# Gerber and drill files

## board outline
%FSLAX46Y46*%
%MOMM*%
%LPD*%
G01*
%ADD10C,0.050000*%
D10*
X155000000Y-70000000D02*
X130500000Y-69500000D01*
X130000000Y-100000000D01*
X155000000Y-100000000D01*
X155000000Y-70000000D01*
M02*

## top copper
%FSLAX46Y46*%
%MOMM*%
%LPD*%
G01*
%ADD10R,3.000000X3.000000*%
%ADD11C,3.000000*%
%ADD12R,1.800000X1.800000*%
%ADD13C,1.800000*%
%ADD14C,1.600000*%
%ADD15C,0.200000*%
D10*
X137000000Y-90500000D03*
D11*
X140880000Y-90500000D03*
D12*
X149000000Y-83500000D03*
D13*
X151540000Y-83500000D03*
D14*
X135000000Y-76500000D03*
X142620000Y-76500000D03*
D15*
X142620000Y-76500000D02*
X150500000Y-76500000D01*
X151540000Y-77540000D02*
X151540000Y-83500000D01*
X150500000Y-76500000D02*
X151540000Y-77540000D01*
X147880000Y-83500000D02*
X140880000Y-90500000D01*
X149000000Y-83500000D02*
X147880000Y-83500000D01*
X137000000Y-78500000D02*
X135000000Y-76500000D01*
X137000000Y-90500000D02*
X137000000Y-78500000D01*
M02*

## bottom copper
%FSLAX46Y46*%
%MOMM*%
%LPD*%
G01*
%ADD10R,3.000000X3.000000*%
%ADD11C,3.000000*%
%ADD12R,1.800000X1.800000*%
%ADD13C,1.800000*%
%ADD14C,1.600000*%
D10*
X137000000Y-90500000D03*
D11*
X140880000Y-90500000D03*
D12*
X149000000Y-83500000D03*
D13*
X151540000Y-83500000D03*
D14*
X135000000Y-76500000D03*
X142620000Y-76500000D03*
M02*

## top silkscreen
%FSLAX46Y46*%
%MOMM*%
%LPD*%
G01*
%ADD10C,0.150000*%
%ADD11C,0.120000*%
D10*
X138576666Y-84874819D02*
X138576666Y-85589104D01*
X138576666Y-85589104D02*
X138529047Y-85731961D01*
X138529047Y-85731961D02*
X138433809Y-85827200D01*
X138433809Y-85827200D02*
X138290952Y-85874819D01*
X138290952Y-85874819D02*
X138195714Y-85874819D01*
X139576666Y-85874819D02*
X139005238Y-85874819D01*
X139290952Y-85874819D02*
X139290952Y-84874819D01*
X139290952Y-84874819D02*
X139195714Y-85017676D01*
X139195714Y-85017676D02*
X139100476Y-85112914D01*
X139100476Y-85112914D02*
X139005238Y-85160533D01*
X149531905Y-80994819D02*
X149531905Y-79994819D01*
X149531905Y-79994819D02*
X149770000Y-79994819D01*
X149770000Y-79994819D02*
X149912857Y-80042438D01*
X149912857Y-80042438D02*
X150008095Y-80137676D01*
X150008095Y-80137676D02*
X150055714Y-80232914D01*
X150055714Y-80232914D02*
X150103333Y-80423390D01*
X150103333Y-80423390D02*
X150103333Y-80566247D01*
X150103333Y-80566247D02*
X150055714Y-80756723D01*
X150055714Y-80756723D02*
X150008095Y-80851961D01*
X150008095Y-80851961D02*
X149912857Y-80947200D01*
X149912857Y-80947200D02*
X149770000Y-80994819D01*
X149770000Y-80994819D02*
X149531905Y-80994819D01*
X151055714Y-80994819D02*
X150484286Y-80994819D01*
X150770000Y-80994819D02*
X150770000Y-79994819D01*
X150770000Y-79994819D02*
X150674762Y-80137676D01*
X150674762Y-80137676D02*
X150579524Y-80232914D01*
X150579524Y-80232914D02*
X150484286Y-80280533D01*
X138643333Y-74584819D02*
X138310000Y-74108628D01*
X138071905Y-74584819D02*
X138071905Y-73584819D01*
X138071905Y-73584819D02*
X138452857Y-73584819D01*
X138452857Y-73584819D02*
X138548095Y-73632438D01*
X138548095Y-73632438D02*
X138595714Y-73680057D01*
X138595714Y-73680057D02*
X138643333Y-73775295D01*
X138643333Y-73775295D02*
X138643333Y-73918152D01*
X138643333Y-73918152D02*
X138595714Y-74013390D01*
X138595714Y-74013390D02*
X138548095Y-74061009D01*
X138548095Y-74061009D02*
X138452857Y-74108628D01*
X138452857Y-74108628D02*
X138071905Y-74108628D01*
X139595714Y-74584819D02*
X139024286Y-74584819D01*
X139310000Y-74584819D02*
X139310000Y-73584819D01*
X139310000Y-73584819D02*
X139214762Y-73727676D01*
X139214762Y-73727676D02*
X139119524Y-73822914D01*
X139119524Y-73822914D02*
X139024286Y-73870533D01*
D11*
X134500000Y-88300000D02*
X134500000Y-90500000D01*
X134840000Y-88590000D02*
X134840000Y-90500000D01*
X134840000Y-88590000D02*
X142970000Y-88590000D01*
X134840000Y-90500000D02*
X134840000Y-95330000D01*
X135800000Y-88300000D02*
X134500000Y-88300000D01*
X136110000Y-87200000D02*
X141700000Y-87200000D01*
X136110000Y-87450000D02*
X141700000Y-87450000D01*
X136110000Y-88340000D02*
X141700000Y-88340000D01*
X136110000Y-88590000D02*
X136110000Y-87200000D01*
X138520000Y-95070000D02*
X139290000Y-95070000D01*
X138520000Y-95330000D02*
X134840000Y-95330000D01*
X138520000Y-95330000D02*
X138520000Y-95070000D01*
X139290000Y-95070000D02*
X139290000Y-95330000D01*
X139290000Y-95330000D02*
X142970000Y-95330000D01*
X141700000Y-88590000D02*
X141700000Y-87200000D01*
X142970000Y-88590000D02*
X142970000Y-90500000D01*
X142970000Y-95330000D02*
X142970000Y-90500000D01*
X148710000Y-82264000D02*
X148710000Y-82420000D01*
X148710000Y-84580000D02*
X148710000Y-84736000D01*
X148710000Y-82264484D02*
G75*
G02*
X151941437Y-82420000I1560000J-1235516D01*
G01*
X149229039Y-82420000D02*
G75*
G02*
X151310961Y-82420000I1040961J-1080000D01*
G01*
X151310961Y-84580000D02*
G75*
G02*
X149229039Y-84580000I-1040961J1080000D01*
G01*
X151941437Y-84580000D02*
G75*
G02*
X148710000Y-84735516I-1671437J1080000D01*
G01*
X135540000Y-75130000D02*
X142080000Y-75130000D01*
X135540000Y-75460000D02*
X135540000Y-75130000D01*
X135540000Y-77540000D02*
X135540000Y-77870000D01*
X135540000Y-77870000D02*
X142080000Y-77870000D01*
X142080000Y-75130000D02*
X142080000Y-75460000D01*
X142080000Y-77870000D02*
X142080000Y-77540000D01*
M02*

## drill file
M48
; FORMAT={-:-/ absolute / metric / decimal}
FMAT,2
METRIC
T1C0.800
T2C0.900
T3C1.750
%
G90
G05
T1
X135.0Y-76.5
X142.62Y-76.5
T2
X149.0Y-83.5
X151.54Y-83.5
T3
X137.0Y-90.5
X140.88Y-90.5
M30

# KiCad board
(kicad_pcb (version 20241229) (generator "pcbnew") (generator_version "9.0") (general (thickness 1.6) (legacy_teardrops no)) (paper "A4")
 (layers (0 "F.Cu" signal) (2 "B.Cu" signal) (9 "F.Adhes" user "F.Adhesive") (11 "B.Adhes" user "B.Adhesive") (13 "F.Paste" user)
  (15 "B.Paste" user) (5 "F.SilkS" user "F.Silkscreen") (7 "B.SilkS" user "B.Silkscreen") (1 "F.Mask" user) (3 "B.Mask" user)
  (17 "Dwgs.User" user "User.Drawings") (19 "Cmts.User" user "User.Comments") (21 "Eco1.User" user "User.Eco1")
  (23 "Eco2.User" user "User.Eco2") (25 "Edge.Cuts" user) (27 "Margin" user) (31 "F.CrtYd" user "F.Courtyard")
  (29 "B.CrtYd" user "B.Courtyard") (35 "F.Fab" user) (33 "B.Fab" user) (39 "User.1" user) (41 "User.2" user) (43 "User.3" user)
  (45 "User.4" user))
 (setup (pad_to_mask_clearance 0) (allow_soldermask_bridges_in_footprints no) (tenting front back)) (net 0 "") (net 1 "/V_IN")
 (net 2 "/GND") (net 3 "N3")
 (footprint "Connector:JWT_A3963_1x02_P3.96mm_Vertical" (layer "F.Cu") (at 137 90.5)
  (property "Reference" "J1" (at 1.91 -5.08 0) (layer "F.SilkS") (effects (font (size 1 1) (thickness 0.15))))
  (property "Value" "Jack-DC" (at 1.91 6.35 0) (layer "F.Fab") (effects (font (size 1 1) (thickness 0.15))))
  (fp_line (start -2.5 -2.2) (end -2.5 0) (stroke (width 0.12) (type solid)) (layer "F.SilkS"))
  (fp_line (start -2.16 -1.91) (end -2.16 0) (stroke (width 0.12) (type solid)) (layer "F.SilkS"))
  (fp_line (start -2.16 -1.91) (end 5.97 -1.91) (stroke (width 0.12) (type solid)) (layer "F.SilkS"))
  (fp_line (start -2.16 0) (end -2.16 4.83) (stroke (width 0.12) (type solid)) (layer "F.SilkS"))
  (fp_line (start -1.2 -2.2) (end -2.5 -2.2) (stroke (width 0.12) (type solid)) (layer "F.SilkS"))
  (fp_line (start -0.89 -3.3) (end 4.7 -3.3) (stroke (width 0.12) (type solid)) (layer "F.SilkS"))
  (fp_line (start -0.89 -3.05) (end 4.7 -3.05) (stroke (width 0.12) (type solid)) (layer "F.SilkS"))
  (fp_line (start -0.89 -2.16) (end 4.7 -2.16) (stroke (width 0.12) (type solid)) (layer "F.SilkS"))
  (fp_line (start -0.89 -1.91) (end -0.89 -3.3) (stroke (width 0.12) (type solid)) (layer "F.SilkS"))
  (fp_line (start 1.52 4.57) (end 2.29 4.57) (stroke (width 0.12) (type solid)) (layer "F.SilkS"))
  (fp_line (start 1.52 4.83) (end -2.16 4.83) (stroke (width 0.12) (type solid)) (layer "F.SilkS"))
  (fp_line (start 1.52 4.83) (end 1.52 4.57) (stroke (width 0.12) (type solid)) (layer "F.SilkS"))
  (fp_line (start 2.29 4.57) (end 2.29 4.83) (stroke (width 0.12) (type solid)) (layer "F.SilkS"))
  (fp_line (start 2.29 4.83) (end 5.97 4.83) (stroke (width 0.12) (type solid)) (layer "F.SilkS"))
  (fp_line (start 4.7 -1.91) (end 4.7 -3.3) (stroke (width 0.12) (type solid)) (layer "F.SilkS"))
  (fp_line (start 5.97 -1.91) (end 5.97 0) (stroke (width 0.12) (type solid)) (layer "F.SilkS"))
  (fp_line (start 5.97 4.83) (end 5.97 0) (stroke (width 0.12) (type solid)) (layer "F.SilkS"))
  (pad "1" thru_hole rect (at 0 0) (size 3 3) (drill 1.75) (layers "*.Cu" "*.Mask") (remove_unused_layers no) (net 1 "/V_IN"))
  (pad "2" thru_hole circle (at 3.88 0) (size 3 3) (drill 1.75) (layers "*.Cu" "*.Mask") (remove_unused_layers no) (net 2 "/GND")))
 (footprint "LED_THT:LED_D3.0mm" (layer "F.Cu") (at 149 83.5)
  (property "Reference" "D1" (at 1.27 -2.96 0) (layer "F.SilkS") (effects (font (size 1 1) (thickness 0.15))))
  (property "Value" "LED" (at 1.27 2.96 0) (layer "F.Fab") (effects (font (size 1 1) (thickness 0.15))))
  (fp_line (start -0.29 -1.236) (end -0.29 -1.08) (stroke (width 0.12) (type solid)) (layer "F.SilkS"))
  (fp_line (start -0.29 1.08) (end -0.29 1.236) (stroke (width 0.12) (type solid)) (layer "F.SilkS"))
  (fp_arc (start -0.29 -1.235516) (mid 1.36566 -1.987699) (end 2.941437 -1.08) (stroke (width 0.12) (type solid)) (layer "F.SilkS"))
  (fp_arc (start 0.229039 -1.08) (mid 1.27 -1.5) (end 2.310961 -1.08) (stroke (width 0.12) (type solid)) (layer "F.SilkS"))
  (fp_arc (start 2.310961 1.08) (mid 1.27 1.5) (end 0.229039 1.08) (stroke (width 0.12) (type solid)) (layer "F.SilkS"))
  (fp_arc (start 2.941437 1.08) (mid 1.36566 1.987699) (end -0.29 1.235516) (stroke (width 0.12) (type solid)) (layer "F.SilkS"))
  (pad "1" thru_hole rect (at 0 0) (size 1.8 1.8) (drill 0.9) (layers "*.Cu" "*.Mask") (remove_unused_layers no) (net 2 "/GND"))
  (pad "2" thru_hole circle (at 2.54 0) (size 1.8 1.8) (drill 0.9) (layers "*.Cu" "*.Mask") (remove_unused_layers no) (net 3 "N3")))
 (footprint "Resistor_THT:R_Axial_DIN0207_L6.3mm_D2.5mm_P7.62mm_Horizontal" (layer "F.Cu") (at 135 76.5)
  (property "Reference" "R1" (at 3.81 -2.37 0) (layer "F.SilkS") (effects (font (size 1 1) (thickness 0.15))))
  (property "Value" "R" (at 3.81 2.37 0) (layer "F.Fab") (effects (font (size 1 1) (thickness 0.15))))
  (fp_line (start 0.54 -1.37) (end 7.08 -1.37) (stroke (width 0.12) (type solid)) (layer "F.SilkS"))
  (fp_line (start 0.54 -1.04) (end 0.54 -1.37) (stroke (width 0.12) (type solid)) (layer "F.SilkS"))
  (fp_line (start 0.54 1.04) (end 0.54 1.37) (stroke (width 0.12) (type solid)) (layer "F.SilkS"))
  (fp_line (start 0.54 1.37) (end 7.08 1.37) (stroke (width 0.12) (type solid)) (layer "F.SilkS"))
  (fp_line (start 7.08 -1.37) (end 7.08 -1.04) (stroke (width 0.12) (type solid)) (layer "F.SilkS"))
  (fp_line (start 7.08 1.37) (end 7.08 1.04) (stroke (width 0.12) (type solid)) (layer "F.SilkS"))
  (pad "1" thru_hole circle (at 0 0) (size 1.6 1.6) (drill 0.8) (layers "*.Cu" "*.Mask") (remove_unused_layers no) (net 1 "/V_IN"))
  (pad "2" thru_hole circle (at 7.62 0) (size 1.6 1.6) (drill 0.8) (layers "*.Cu" "*.Mask") (remove_unused_layers no) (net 3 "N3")))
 (gr_poly (pts (xy 155 70) (xy 130.5 69.5) (xy 130 100) (xy 155 100)) (stroke (width 0.05) (type solid)) (fill no) (layer "Edge.Cuts"))
 (segment (start 142.62 76.5) (end 150.5 76.5) (width 0.2) (layer "F.Cu") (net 3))
 (segment (start 151.54 77.54) (end 151.54 83.5) (width 0.2) (layer "F.Cu") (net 3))
 (segment (start 150.5 76.5) (end 151.54 77.54) (width 0.2) (layer "F.Cu") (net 3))
 (segment (start 147.88 83.5) (end 140.88 90.5) (width 0.2) (layer "F.Cu") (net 2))
 (segment (start 149 83.5) (end 147.88 83.5) (width 0.2) (layer "F.Cu") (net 2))
 (segment (start 137 78.5) (end 135 76.5) (width 0.2) (layer "F.Cu") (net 1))
 (segment (start 137 90.5) (end 137 78.5) (width 0.2) (layer "F.Cu") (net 1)))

